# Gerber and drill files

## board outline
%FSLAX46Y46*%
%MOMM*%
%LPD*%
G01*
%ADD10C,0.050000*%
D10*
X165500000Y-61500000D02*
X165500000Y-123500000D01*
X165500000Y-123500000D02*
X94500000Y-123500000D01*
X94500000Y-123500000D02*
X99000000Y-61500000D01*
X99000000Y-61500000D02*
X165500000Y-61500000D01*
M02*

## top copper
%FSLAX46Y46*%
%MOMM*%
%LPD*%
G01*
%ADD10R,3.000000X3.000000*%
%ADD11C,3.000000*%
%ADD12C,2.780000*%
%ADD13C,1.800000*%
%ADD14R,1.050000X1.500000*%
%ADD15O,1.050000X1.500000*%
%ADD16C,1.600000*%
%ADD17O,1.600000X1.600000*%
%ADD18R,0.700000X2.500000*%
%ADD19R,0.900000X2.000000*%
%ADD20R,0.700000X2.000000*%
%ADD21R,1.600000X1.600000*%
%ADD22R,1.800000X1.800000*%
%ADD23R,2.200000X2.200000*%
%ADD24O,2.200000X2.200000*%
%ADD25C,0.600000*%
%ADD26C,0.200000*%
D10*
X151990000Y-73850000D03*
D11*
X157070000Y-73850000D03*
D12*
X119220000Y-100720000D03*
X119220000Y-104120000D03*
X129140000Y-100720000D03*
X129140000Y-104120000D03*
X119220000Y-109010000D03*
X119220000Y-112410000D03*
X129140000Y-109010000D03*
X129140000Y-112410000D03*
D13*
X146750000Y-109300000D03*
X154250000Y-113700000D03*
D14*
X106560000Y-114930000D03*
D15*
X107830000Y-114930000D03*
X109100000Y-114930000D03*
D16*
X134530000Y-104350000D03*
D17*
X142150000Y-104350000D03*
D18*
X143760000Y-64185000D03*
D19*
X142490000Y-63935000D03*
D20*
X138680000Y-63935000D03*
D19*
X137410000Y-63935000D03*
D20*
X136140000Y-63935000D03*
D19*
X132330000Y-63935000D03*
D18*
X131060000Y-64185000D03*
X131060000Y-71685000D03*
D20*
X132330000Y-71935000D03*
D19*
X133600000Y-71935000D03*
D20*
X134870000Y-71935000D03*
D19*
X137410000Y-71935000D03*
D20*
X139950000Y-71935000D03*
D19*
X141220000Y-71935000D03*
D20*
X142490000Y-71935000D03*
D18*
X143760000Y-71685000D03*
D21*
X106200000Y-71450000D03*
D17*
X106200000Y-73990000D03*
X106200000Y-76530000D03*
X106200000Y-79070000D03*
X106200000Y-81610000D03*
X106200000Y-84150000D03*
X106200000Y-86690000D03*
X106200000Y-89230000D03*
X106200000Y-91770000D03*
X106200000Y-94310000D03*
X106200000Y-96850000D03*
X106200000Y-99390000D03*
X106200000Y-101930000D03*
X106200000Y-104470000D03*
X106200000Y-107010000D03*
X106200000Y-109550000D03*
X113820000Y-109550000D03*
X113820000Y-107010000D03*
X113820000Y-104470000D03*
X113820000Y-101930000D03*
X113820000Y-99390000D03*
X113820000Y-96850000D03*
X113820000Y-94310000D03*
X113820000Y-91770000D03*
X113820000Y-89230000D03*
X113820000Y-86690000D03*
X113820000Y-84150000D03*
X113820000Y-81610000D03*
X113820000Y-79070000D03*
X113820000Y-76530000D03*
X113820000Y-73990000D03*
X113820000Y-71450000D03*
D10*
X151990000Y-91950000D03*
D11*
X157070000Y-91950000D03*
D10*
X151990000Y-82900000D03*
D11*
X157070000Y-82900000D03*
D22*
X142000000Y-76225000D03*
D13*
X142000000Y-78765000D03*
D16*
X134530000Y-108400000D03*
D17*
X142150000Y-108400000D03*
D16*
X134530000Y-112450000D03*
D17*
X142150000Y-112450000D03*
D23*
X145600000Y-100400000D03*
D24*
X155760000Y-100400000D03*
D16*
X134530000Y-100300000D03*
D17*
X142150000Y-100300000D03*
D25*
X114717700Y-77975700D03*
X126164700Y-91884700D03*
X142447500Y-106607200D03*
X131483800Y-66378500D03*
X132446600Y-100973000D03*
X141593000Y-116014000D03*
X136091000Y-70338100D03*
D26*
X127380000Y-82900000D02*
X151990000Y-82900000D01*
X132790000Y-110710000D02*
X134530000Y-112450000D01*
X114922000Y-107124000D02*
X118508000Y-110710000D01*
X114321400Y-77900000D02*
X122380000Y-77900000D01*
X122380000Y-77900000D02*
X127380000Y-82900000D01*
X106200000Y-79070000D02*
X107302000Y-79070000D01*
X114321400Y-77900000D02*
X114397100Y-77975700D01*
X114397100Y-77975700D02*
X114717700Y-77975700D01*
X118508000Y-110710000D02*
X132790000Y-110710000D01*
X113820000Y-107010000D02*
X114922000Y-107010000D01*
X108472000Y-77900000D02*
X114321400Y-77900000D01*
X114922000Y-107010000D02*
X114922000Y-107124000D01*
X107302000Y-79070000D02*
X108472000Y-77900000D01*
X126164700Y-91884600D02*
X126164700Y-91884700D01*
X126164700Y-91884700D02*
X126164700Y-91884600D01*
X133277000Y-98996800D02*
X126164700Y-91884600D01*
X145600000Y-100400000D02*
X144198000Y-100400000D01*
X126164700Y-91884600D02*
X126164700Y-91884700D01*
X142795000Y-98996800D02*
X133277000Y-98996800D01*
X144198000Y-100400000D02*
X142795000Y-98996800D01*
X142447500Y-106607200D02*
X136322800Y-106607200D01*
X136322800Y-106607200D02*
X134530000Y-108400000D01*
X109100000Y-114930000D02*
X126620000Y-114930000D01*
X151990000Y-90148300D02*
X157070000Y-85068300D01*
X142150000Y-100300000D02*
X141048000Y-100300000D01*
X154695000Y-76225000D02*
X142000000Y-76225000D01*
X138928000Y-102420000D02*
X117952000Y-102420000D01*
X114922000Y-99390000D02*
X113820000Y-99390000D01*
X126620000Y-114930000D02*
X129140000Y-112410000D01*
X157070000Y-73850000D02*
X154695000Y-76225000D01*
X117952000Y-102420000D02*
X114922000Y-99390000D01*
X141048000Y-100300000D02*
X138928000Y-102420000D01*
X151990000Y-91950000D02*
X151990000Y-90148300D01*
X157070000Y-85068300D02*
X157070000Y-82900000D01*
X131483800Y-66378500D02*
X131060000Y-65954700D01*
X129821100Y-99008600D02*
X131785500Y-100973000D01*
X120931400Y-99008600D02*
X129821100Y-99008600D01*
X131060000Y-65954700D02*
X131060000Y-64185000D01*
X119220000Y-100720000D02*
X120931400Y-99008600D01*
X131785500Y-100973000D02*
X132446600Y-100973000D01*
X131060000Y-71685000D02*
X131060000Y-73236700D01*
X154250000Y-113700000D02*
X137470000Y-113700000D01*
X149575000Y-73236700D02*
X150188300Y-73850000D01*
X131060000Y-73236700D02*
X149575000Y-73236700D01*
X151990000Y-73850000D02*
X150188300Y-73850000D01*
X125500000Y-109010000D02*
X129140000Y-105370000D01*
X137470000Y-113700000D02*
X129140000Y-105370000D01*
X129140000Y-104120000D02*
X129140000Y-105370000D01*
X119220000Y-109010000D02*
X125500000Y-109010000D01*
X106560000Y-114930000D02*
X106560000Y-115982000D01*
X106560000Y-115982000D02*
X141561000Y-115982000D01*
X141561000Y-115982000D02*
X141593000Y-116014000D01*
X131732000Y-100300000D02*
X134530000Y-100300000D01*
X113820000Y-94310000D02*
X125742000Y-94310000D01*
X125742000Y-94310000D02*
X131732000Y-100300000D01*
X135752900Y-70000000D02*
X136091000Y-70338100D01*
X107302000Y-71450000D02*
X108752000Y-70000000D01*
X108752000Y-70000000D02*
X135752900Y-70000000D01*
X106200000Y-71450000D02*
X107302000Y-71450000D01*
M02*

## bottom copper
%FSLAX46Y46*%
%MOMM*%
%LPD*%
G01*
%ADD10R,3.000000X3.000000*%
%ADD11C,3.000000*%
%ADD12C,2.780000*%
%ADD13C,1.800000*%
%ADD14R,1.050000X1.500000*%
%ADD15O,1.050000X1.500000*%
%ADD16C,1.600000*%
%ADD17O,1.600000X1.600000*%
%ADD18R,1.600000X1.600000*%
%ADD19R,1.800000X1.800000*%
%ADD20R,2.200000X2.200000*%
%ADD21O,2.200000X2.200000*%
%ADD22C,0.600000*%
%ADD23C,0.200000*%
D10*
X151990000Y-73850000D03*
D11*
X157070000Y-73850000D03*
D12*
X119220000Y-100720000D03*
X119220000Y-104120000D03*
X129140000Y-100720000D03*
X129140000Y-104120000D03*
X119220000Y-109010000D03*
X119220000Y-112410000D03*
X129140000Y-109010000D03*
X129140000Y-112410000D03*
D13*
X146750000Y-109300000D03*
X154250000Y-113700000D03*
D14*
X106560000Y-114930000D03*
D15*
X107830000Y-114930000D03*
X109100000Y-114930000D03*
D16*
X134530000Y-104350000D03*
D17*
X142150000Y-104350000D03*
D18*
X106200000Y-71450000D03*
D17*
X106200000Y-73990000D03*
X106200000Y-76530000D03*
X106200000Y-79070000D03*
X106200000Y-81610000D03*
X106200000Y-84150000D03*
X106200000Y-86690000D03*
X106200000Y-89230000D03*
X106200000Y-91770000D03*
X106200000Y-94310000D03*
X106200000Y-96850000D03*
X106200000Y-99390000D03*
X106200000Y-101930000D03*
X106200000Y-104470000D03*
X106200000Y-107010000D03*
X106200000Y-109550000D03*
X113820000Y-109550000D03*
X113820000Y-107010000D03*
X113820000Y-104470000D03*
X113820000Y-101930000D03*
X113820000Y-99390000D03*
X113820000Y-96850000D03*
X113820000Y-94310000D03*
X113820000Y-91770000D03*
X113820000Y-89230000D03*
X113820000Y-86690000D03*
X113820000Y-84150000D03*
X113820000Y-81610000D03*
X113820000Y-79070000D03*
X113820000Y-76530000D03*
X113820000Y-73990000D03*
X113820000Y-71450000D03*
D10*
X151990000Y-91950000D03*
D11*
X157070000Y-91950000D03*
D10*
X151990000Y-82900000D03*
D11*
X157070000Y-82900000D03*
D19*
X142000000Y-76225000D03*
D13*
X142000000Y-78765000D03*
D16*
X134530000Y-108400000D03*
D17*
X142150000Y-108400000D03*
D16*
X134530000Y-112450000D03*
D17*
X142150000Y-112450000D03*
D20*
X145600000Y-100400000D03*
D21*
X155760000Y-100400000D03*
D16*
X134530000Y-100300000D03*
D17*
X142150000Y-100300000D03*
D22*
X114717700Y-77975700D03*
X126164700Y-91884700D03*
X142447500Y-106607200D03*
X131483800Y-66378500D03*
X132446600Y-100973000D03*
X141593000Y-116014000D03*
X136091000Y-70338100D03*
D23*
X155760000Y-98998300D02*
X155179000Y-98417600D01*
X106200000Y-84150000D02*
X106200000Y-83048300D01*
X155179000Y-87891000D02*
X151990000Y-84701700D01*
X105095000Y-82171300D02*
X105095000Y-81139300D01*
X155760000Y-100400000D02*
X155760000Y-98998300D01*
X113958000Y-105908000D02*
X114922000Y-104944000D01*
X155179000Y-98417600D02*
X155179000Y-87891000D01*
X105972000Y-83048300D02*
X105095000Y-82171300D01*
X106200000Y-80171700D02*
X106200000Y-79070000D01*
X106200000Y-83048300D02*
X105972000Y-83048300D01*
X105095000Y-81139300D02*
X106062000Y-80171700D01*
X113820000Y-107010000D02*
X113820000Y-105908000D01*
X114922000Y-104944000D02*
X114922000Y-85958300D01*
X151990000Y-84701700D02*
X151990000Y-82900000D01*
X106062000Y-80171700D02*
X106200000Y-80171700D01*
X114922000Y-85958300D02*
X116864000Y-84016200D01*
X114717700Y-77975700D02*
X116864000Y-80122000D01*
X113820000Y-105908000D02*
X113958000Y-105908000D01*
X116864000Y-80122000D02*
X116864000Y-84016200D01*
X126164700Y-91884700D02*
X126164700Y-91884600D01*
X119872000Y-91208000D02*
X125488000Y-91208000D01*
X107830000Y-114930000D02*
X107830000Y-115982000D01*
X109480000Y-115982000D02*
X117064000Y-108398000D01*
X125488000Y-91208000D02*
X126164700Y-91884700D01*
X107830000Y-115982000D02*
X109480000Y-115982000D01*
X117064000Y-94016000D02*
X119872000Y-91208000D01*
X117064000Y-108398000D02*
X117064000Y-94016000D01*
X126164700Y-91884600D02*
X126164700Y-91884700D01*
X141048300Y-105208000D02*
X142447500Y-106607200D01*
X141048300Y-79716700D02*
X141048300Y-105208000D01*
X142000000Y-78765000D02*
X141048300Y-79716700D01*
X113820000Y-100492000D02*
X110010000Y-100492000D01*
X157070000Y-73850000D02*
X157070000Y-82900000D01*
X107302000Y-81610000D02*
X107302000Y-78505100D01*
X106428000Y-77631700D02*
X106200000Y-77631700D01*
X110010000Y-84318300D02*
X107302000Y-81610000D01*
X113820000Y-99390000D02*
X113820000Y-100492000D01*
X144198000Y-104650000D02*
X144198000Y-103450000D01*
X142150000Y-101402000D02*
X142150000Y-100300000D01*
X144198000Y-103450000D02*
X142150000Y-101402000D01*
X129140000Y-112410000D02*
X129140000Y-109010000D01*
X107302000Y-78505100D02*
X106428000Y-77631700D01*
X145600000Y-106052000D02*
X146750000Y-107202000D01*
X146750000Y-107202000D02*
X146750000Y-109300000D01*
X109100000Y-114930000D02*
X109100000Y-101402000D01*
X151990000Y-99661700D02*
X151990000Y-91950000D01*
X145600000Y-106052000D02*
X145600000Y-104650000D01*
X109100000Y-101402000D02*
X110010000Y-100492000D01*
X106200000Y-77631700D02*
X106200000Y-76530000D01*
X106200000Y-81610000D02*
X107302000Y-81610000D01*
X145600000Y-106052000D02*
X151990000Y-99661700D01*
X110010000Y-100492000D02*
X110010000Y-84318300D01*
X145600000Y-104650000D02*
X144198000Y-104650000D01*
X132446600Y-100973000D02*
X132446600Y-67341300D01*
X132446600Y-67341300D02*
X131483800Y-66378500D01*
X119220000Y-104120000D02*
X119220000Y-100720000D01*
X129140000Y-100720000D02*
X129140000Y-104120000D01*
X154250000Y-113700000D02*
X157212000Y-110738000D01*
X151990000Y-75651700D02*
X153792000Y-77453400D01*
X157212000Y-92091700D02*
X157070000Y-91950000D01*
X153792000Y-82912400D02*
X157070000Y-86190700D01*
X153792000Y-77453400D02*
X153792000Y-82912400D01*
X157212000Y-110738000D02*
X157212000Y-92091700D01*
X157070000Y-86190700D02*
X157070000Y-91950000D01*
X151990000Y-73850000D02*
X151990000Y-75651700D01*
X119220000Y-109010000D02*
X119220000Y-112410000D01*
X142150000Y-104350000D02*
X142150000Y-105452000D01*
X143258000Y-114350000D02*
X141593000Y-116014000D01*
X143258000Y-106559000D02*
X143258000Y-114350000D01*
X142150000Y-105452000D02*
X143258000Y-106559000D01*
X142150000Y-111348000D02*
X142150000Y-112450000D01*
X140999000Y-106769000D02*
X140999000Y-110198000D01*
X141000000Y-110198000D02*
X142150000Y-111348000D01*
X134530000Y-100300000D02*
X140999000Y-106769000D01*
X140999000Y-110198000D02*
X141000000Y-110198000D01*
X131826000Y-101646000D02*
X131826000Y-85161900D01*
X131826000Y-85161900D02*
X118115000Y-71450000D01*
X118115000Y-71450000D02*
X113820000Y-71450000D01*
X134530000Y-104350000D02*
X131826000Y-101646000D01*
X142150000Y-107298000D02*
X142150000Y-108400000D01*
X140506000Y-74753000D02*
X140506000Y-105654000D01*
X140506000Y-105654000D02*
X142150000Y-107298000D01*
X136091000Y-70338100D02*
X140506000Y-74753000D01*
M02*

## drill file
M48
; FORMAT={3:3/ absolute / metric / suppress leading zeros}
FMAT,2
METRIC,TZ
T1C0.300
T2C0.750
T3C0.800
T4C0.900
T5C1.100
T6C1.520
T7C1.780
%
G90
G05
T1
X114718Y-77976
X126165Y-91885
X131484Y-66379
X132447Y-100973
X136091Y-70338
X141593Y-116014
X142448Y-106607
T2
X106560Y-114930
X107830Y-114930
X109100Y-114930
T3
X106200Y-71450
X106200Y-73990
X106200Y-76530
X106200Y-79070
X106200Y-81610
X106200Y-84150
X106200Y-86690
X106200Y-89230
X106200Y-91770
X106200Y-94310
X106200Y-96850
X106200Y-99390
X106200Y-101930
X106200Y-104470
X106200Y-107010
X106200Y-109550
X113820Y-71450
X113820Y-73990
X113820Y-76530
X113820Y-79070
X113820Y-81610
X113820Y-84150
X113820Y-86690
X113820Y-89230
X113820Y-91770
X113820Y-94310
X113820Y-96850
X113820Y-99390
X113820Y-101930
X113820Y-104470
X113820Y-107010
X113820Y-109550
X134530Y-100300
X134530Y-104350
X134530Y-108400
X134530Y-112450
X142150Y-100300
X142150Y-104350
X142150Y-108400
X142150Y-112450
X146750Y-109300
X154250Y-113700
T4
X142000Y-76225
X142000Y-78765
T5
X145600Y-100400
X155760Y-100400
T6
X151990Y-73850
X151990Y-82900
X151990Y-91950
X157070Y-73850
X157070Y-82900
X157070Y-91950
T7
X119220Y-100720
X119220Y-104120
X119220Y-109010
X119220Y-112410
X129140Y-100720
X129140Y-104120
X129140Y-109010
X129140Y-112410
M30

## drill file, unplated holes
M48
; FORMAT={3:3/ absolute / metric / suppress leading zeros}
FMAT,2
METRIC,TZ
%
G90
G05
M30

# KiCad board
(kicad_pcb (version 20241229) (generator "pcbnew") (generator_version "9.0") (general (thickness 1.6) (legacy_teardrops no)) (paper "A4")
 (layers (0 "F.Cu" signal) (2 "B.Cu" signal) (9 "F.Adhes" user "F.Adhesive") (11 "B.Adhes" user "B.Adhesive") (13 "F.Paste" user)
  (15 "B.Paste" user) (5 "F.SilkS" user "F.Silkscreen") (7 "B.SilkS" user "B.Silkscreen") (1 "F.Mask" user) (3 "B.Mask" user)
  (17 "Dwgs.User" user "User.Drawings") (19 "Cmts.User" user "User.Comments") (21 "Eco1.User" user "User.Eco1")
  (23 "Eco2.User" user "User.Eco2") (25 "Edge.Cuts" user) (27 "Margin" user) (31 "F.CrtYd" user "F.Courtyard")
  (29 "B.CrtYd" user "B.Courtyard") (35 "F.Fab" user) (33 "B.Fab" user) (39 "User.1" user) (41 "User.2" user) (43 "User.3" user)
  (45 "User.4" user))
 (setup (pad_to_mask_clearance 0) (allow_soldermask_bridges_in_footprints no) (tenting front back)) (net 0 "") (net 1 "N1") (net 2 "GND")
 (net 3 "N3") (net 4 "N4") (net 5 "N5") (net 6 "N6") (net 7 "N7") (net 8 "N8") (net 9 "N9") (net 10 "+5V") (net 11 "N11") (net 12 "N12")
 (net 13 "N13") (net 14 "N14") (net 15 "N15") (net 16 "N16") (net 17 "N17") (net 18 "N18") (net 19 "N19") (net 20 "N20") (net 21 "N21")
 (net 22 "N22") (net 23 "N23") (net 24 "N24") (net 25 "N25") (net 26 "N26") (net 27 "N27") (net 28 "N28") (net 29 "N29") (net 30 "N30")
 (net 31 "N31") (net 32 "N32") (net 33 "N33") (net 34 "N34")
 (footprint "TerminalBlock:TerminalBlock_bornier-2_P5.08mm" (layer "F.Cu") (at 151.99 73.85)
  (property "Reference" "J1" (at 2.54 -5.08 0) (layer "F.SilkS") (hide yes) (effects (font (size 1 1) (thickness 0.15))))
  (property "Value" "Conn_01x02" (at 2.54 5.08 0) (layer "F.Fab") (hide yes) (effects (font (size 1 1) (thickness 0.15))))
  (pad "1" thru_hole rect (at 0 0) (size 3 3) (drill 1.52) (layers "*.Cu" "*.Mask") (remove_unused_layers no) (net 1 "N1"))
  (pad "2" thru_hole circle (at 5.08 0) (size 3 3) (drill 1.52) (layers "*.Cu" "*.Mask") (remove_unused_layers no) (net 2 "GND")))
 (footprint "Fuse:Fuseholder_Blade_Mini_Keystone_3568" (layer "F.Cu") (at 119.22 100.72)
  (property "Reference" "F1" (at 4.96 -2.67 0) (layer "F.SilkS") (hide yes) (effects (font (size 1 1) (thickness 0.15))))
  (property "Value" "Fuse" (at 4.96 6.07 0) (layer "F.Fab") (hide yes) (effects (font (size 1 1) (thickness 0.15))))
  (pad "1" thru_hole circle (at 0 0) (size 2.78 2.78) (drill 1.78) (layers "*.Cu" "*.Mask") (remove_unused_layers no) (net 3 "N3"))
  (pad "1" thru_hole circle (at 0 3.4) (size 2.78 2.78) (drill 1.78) (layers "*.Cu" "*.Mask") (remove_unused_layers no) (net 3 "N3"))
  (pad "2" thru_hole circle (at 9.92 0) (size 2.78 2.78) (drill 1.78) (layers "*.Cu" "*.Mask") (remove_unused_layers no) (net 1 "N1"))
  (pad "2" thru_hole circle (at 9.92 3.4) (size 2.78 2.78) (drill 1.78) (layers "*.Cu" "*.Mask") (remove_unused_layers no) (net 1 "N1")))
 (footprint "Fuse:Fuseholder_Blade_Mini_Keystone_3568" (layer "F.Cu") (at 119.22 109.01)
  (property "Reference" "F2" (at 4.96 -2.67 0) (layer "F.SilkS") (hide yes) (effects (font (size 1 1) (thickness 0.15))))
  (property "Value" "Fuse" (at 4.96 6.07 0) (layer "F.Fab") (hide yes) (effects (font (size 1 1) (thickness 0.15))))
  (pad "1" thru_hole circle (at 0 0) (size 2.78 2.78) (drill 1.78) (layers "*.Cu" "*.Mask") (remove_unused_layers no) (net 1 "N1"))
  (pad "1" thru_hole circle (at 0 3.4) (size 2.78 2.78) (drill 1.78) (layers "*.Cu" "*.Mask") (remove_unused_layers no) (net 1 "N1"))
  (pad "2" thru_hole circle (at 9.92 0) (size 2.78 2.78) (drill 1.78) (layers "*.Cu" "*.Mask") (remove_unused_layers no) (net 2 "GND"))
  (pad "2" thru_hole circle (at 9.92 3.4) (size 2.78 2.78) (drill 1.78) (layers "*.Cu" "*.Mask") (remove_unused_layers no) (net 2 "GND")))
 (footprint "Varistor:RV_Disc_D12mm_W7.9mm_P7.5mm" (layer "F.Cu") (at 146.75 109.3)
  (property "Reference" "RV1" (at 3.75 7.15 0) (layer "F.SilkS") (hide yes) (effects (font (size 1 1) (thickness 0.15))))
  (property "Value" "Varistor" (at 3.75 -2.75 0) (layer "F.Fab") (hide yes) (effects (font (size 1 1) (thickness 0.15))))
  (pad "1" thru_hole circle (at 0 0) (size 1.8 1.8) (drill 0.8) (layers "*.Cu" "*.Mask") (remove_unused_layers no) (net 2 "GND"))
  (pad "2" thru_hole circle (at 7.5 4.4) (size 1.8 1.8) (drill 0.8) (layers "*.Cu" "*.Mask") (remove_unused_layers no) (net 1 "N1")))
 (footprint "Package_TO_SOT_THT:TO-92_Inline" (layer "F.Cu") (at 106.56 114.93)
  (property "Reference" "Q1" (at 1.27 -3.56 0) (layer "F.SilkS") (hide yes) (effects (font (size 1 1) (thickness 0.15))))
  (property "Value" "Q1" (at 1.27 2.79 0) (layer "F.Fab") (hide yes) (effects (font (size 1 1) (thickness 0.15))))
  (pad "1" thru_hole rect (at 0 0) (size 1.05 1.5) (drill 0.75) (layers "*.Cu" "*.Mask") (remove_unused_layers no) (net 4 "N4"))
  (pad "2" thru_hole oval (at 1.27 0) (size 1.05 1.5) (drill 0.75) (layers "*.Cu" "*.Mask") (remove_unused_layers no) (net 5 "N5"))
  (pad "3" thru_hole oval (at 2.54 0) (size 1.05 1.5) (drill 0.75) (layers "*.Cu" "*.Mask") (remove_unused_layers no) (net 2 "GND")))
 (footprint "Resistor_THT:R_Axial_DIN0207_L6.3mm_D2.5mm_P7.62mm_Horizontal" (layer "F.Cu") (at 134.53 104.35)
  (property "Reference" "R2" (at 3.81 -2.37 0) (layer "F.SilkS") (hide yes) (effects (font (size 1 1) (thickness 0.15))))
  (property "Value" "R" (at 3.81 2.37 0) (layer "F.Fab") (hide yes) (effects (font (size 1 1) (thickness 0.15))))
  (pad "1" thru_hole circle (at 0 0) (size 1.6 1.6) (drill 0.8) (layers "*.Cu" "*.Mask") (remove_unused_layers no) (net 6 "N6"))
  (pad "2" thru_hole oval (at 7.62 0) (size 1.6 1.6) (drill 0.8) (layers "*.Cu" "*.Mask") (remove_unused_layers no) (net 4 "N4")))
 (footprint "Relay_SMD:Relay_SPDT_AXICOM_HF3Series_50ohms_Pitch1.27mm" (layer "F.Cu") (at 137.41 67.935 -90)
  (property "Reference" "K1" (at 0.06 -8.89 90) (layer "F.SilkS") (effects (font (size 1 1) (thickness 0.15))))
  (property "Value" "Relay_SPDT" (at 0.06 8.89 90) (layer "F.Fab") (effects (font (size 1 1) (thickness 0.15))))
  (pad "1" smd rect (at -3.75 -6.35 270) (size 2.5 0.7) (layers "F.Cu" "F.Mask" "F.Paste"))
  (pad "2" smd rect (at -4 -5.08 270) (size 2 0.9) (layers "F.Cu" "F.Mask" "F.Paste"))
  (pad "5" smd rect (at -4 -1.27 270) (size 2 0.7) (layers "F.Cu" "F.Mask" "F.Paste"))
  (pad "6" smd rect (at -4 0 270) (size 2 0.9) (layers "F.Cu" "F.Mask" "F.Paste"))
  (pad "7" smd rect (at -4 1.27 270) (size 2 0.7) (layers "F.Cu" "F.Mask" "F.Paste"))
  (pad "10" smd rect (at -4 5.08 270) (size 2 0.9) (layers "F.Cu" "F.Mask" "F.Paste"))
  (pad "11" smd rect (at -3.75 6.35 270) (size 2.5 0.7) (layers "F.Cu" "F.Mask" "F.Paste") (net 3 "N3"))
  (pad "12" smd rect (at 3.75 6.35 270) (size 2.5 0.7) (layers "F.Cu" "F.Mask" "F.Paste") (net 1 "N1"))
  (pad "13" smd rect (at 4 5.08 270) (size 2 0.7) (layers "F.Cu" "F.Mask" "F.Paste"))
  (pad "14" smd rect (at 4 3.81 270) (size 2 0.9) (layers "F.Cu" "F.Mask" "F.Paste") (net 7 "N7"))
  (pad "15" smd rect (at 4 2.54 270) (size 2 0.7) (layers "F.Cu" "F.Mask" "F.Paste"))
  (pad "17" smd rect (at 4 0 270) (size 2 0.9) (layers "F.Cu" "F.Mask" "F.Paste"))
  (pad "19" smd rect (at 4 -2.54 270) (size 2 0.7) (layers "F.Cu" "F.Mask" "F.Paste"))
  (pad "20" smd rect (at 4 -3.81 270) (size 2 0.9) (layers "F.Cu" "F.Mask" "F.Paste"))
  (pad "21" smd rect (at 4 -5.08 270) (size 2 0.7) (layers "F.Cu" "F.Mask" "F.Paste"))
  (pad "22" smd rect (at 3.75 -6.35 270) (size 2.5 0.7) (layers "F.Cu" "F.Mask" "F.Paste")))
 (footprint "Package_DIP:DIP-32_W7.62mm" (layer "F.Cu") (at 106.2 71.45)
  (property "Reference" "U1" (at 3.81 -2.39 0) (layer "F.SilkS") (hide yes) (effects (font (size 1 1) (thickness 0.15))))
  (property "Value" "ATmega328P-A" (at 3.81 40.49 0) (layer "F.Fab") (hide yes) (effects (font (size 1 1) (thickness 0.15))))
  (pad "1" thru_hole rect (at 0 0) (size 1.6 1.6) (drill 0.8) (layers "*.Cu" "*.Mask") (remove_unused_layers no) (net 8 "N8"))
  (pad "2" thru_hole oval (at 0 2.54) (size 1.6 1.6) (drill 0.8) (layers "*.Cu" "*.Mask") (remove_unused_layers no) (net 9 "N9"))
  (pad "3" thru_hole oval (at 0 5.08) (size 1.6 1.6) (drill 0.8) (layers "*.Cu" "*.Mask") (remove_unused_layers no) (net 2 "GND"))
  (pad "4" thru_hole oval (at 0 7.62) (size 1.6 1.6) (drill 0.8) (layers "*.Cu" "*.Mask") (remove_unused_layers no) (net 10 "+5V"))
  (pad "5" thru_hole oval (at 0 10.16) (size 1.6 1.6) (drill 0.8) (layers "*.Cu" "*.Mask") (remove_unused_layers no) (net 2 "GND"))
  (pad "6" thru_hole oval (at 0 12.7) (size 1.6 1.6) (drill 0.8) (layers "*.Cu" "*.Mask") (remove_unused_layers no) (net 10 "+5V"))
  (pad "7" thru_hole oval (at 0 15.24) (size 1.6 1.6) (drill 0.8) (layers "*.Cu" "*.Mask") (remove_unused_layers no) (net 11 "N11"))
  (pad "8" thru_hole oval (at 0 17.78) (size 1.6 1.6) (drill 0.8) (layers "*.Cu" "*.Mask") (remove_unused_layers no) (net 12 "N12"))
  (pad "9" thru_hole oval (at 0 20.32) (size 1.6 1.6) (drill 0.8) (layers "*.Cu" "*.Mask") (remove_unused_layers no) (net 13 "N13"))
  (pad "10" thru_hole oval (at 0 22.86) (size 1.6 1.6) (drill 0.8) (layers "*.Cu" "*.Mask") (remove_unused_layers no) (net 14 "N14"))
  (pad "11" thru_hole oval (at 0 25.4) (size 1.6 1.6) (drill 0.8) (layers "*.Cu" "*.Mask") (remove_unused_layers no) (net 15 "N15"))
  (pad "12" thru_hole oval (at 0 27.94) (size 1.6 1.6) (drill 0.8) (layers "*.Cu" "*.Mask") (remove_unused_layers no) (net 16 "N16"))
  (pad "13" thru_hole oval (at 0 30.48) (size 1.6 1.6) (drill 0.8) (layers "*.Cu" "*.Mask") (remove_unused_layers no) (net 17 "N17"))
  (pad "14" thru_hole oval (at 0 33.02) (size 1.6 1.6) (drill 0.8) (layers "*.Cu" "*.Mask") (remove_unused_layers no) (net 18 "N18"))
  (pad "15" thru_hole oval (at 0 35.56) (size 1.6 1.6) (drill 0.8) (layers "*.Cu" "*.Mask") (remove_unused_layers no) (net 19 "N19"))
  (pad "16" thru_hole oval (at 0 38.1) (size 1.6 1.6) (drill 0.8) (layers "*.Cu" "*.Mask") (remove_unused_layers no) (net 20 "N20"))
  (pad "17" thru_hole oval (at 7.62 38.1) (size 1.6 1.6) (drill 0.8) (layers "*.Cu" "*.Mask") (remove_unused_layers no) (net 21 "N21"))
  (pad "18" thru_hole oval (at 7.62 35.56) (size 1.6 1.6) (drill 0.8) (layers "*.Cu" "*.Mask") (remove_unused_layers no) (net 10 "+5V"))
  (pad "19" thru_hole oval (at 7.62 33.02) (size 1.6 1.6) (drill 0.8) (layers "*.Cu" "*.Mask") (remove_unused_layers no) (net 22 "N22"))
  (pad "20" thru_hole oval (at 7.62 30.48) (size 1.6 1.6) (drill 0.8) (layers "*.Cu" "*.Mask") (remove_unused_layers no) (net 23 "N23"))
  (pad "21" thru_hole oval (at 7.62 27.94) (size 1.6 1.6) (drill 0.8) (layers "*.Cu" "*.Mask") (remove_unused_layers no) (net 2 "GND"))
  (pad "22" thru_hole oval (at 7.62 25.4) (size 1.6 1.6) (drill 0.8) (layers "*.Cu" "*.Mask") (remove_unused_layers no) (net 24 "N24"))
  (pad "23" thru_hole oval (at 7.62 22.86) (size 1.6 1.6) (drill 0.8) (layers "*.Cu" "*.Mask") (remove_unused_layers no) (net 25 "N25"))
  (pad "24" thru_hole oval (at 7.62 20.32) (size 1.6 1.6) (drill 0.8) (layers "*.Cu" "*.Mask") (remove_unused_layers no) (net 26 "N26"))
  (pad "25" thru_hole oval (at 7.62 17.78) (size 1.6 1.6) (drill 0.8) (layers "*.Cu" "*.Mask") (remove_unused_layers no) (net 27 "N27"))
  (pad "26" thru_hole oval (at 7.62 15.24) (size 1.6 1.6) (drill 0.8) (layers "*.Cu" "*.Mask") (remove_unused_layers no) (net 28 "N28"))
  (pad "27" thru_hole oval (at 7.62 12.7) (size 1.6 1.6) (drill 0.8) (layers "*.Cu" "*.Mask") (remove_unused_layers no) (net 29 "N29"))
  (pad "28" thru_hole oval (at 7.62 10.16) (size 1.6 1.6) (drill 0.8) (layers "*.Cu" "*.Mask") (remove_unused_layers no) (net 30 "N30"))
  (pad "29" thru_hole oval (at 7.62 7.62) (size 1.6 1.6) (drill 0.8) (layers "*.Cu" "*.Mask") (remove_unused_layers no) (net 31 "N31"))
  (pad "30" thru_hole oval (at 7.62 5.08) (size 1.6 1.6) (drill 0.8) (layers "*.Cu" "*.Mask") (remove_unused_layers no) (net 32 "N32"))
  (pad "31" thru_hole oval (at 7.62 2.54) (size 1.6 1.6) (drill 0.8) (layers "*.Cu" "*.Mask") (remove_unused_layers no) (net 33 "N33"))
  (pad "32" thru_hole oval (at 7.62 0) (size 1.6 1.6) (drill 0.8) (layers "*.Cu" "*.Mask") (remove_unused_layers no) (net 6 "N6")))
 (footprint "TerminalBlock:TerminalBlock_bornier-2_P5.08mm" (layer "F.Cu") (at 151.99 91.95)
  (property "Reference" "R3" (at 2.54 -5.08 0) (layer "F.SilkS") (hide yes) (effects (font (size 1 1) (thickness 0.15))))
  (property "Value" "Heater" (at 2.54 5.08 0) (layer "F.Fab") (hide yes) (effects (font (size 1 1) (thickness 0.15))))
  (pad "1" thru_hole rect (at 0 0) (size 3 3) (drill 1.52) (layers "*.Cu" "*.Mask") (remove_unused_layers no) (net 2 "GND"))
  (pad "2" thru_hole circle (at 5.08 0) (size 3 3) (drill 1.52) (layers "*.Cu" "*.Mask") (remove_unused_layers no) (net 1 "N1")))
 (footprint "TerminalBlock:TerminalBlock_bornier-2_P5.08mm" (layer "F.Cu") (at 151.99 82.9)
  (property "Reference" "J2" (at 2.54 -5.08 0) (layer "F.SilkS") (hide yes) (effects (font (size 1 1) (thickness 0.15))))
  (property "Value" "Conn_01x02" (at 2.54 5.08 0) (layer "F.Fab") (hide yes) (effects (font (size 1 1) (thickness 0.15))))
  (pad "1" thru_hole rect (at 0 0) (size 3 3) (drill 1.52) (layers "*.Cu" "*.Mask") (remove_unused_layers no) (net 10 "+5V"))
  (pad "2" thru_hole circle (at 5.08 0) (size 3 3) (drill 1.52) (layers "*.Cu" "*.Mask") (remove_unused_layers no) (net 2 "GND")))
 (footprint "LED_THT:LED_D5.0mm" (layer "F.Cu") (at 142 76.225 -90)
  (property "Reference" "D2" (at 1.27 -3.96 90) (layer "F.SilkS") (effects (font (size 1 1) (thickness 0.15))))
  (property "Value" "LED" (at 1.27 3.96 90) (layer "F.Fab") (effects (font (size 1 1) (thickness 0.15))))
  (pad "1" thru_hole rect (at 0 0 270) (size 1.8 1.8) (drill 0.9) (layers "*.Cu" "*.Mask") (remove_unused_layers no) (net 2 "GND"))
  (pad "2" thru_hole circle (at 2.54 0 270) (size 1.8 1.8) (drill 0.9) (layers "*.Cu" "*.Mask") (remove_unused_layers no) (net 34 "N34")))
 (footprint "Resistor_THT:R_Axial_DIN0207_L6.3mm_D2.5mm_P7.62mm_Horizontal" (layer "F.Cu") (at 134.53 108.4)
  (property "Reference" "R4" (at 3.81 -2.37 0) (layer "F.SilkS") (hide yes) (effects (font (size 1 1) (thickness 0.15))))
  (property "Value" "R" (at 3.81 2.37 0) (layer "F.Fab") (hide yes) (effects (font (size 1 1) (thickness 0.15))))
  (pad "1" thru_hole circle (at 0 0) (size 1.6 1.6) (drill 0.8) (layers "*.Cu" "*.Mask") (remove_unused_layers no) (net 34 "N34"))
  (pad "2" thru_hole oval (at 7.62 0) (size 1.6 1.6) (drill 0.8) (layers "*.Cu" "*.Mask") (remove_unused_layers no) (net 8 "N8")))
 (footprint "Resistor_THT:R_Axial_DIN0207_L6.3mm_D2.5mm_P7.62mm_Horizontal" (layer "F.Cu") (at 134.53 112.45)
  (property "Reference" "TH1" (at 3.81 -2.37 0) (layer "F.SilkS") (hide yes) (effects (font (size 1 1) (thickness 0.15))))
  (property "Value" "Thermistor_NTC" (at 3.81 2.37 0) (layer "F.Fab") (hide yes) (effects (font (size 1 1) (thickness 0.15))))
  (pad "1" thru_hole circle (at 0 0) (size 1.6 1.6) (drill 0.8) (layers "*.Cu" "*.Mask") (remove_unused_layers no) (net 10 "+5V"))
  (pad "2" thru_hole oval (at 7.62 0) (size 1.6 1.6) (drill 0.8) (layers "*.Cu" "*.Mask") (remove_unused_layers no) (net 25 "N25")))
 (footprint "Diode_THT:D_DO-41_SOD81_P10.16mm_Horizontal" (layer "F.Cu") (at 145.6 100.4)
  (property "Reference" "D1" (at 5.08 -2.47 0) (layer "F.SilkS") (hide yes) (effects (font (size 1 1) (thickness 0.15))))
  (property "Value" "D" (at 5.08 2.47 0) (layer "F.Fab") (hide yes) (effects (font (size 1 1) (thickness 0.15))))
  (pad "1" thru_hole rect (at 0 0) (size 2.2 2.2) (drill 1.1) (layers "*.Cu" "*.Mask") (remove_unused_layers no) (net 5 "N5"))
  (pad "2" thru_hole oval (at 10.16 0) (size 2.2 2.2) (drill 1.1) (layers "*.Cu" "*.Mask") (remove_unused_layers no) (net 10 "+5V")))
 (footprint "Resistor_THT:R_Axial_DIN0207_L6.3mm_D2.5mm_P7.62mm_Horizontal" (layer "F.Cu") (at 134.53 100.3)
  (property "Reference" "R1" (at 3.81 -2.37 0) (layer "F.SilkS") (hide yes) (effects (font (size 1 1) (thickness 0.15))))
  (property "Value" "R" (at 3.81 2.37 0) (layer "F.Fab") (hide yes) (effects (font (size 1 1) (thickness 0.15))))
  (pad "1" thru_hole circle (at 0 0) (size 1.6 1.6) (drill 0.8) (layers "*.Cu" "*.Mask") (remove_unused_layers no) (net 25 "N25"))
  (pad "2" thru_hole oval (at 7.62 0) (size 1.6 1.6) (drill 0.8) (layers "*.Cu" "*.Mask") (remove_unused_layers no) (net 2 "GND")))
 (gr_line (start 165.5 61.5) (end 165.5 123.5) (stroke (width 0.05) (type default)) (layer "Edge.Cuts"))
 (gr_line (start 165.5 123.5) (end 94.5 123.5) (stroke (width 0.05) (type default)) (layer "Edge.Cuts"))
 (gr_line (start 94.5 123.5) (end 99 61.5) (stroke (width 0.05) (type default)) (layer "Edge.Cuts"))
 (gr_line (start 99 61.5) (end 165.5 61.5) (stroke (width 0.05) (type default)) (layer "Edge.Cuts"))
 (segment (start 127.38 82.9) (end 151.99 82.9) (width 0.2) (layer "F.Cu") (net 10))
 (segment (start 132.79 110.71) (end 134.53 112.45) (width 0.2) (layer "F.Cu") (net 10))
 (segment (start 114.922 107.124) (end 118.508 110.71) (width 0.2) (layer "F.Cu") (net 10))
 (segment (start 114.3214 77.9) (end 122.38 77.9) (width 0.2) (layer "F.Cu") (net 10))
 (segment (start 122.38 77.9) (end 127.38 82.9) (width 0.2) (layer "F.Cu") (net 10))
 (segment (start 106.2 79.07) (end 107.302 79.07) (width 0.2) (layer "F.Cu") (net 10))
 (segment (start 114.3214 77.9) (end 114.3971 77.9757) (width 0.2) (layer "F.Cu") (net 10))
 (segment (start 114.3971 77.9757) (end 114.7177 77.9757) (width 0.2) (layer "F.Cu") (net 10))
 (segment (start 118.508 110.71) (end 132.79 110.71) (width 0.2) (layer "F.Cu") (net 10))
 (segment (start 113.82 107.01) (end 114.922 107.01) (width 0.2) (layer "F.Cu") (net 10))
 (segment (start 108.472 77.9) (end 114.3214 77.9) (width 0.2) (layer "F.Cu") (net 10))
 (segment (start 114.922 107.01) (end 114.922 107.124) (width 0.2) (layer "F.Cu") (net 10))
 (segment (start 107.302 79.07) (end 108.472 77.9) (width 0.2) (layer "F.Cu") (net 10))
 (via (at 114.7177 77.9757) (size 0.6) (drill 0.3) (layers "F.Cu" "B.Cu") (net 10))
 (segment (start 155.76 98.9983) (end 155.179 98.4176) (width 0.2) (layer "B.Cu") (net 10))
 (segment (start 106.2 84.15) (end 106.2 83.0483) (width 0.2) (layer "B.Cu") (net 10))
 (segment (start 155.179 87.891) (end 151.99 84.7017) (width 0.2) (layer "B.Cu") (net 10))
 (segment (start 105.095 82.1713) (end 105.095 81.1393) (width 0.2) (layer "B.Cu") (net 10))
 (segment (start 155.76 100.4) (end 155.76 98.9983) (width 0.2) (layer "B.Cu") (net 10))
 (segment (start 113.958 105.908) (end 114.922 104.944) (width 0.2) (layer "B.Cu") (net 10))
 (segment (start 155.179 98.4176) (end 155.179 87.891) (width 0.2) (layer "B.Cu") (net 10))
 (segment (start 105.972 83.0483) (end 105.095 82.1713) (width 0.2) (layer "B.Cu") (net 10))
 (segment (start 106.2 80.1717) (end 106.2 79.07) (width 0.2) (layer "B.Cu") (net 10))
 (segment (start 106.2 83.0483) (end 105.972 83.0483) (width 0.2) (layer "B.Cu") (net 10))
 (segment (start 105.095 81.1393) (end 106.062 80.1717) (width 0.2) (layer "B.Cu") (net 10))
 (segment (start 113.82 107.01) (end 113.82 105.908) (width 0.2) (layer "B.Cu") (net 10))
 (segment (start 114.922 104.944) (end 114.922 85.9583) (width 0.2) (layer "B.Cu") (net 10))
 (segment (start 151.99 84.7017) (end 151.99 82.9) (width 0.2) (layer "B.Cu") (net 10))
 (segment (start 106.062 80.1717) (end 106.2 80.1717) (width 0.2) (layer "B.Cu") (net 10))
 (segment (start 114.922 85.9583) (end 116.864 84.0162) (width 0.2) (layer "B.Cu") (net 10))
 (segment (start 114.7177 77.9757) (end 116.864 80.122) (width 0.2) (layer "B.Cu") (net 10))
 (segment (start 113.82 105.908) (end 113.958 105.908) (width 0.2) (layer "B.Cu") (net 10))
 (segment (start 116.864 80.122) (end 116.864 84.0162) (width 0.2) (layer "B.Cu") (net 10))
 (segment (start 126.1647 91.8846) (end 126.1647 91.8847) (width 0.2) (layer "F.Cu") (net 5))
 (segment (start 126.1647 91.8847) (end 126.1647 91.8846) (width 0.2) (layer "F.Cu") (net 5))
 (segment (start 133.277 98.9968) (end 126.1647 91.8846) (width 0.2) (layer "F.Cu") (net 5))
 (segment (start 145.6 100.4) (end 144.198 100.4) (width 0.2) (layer "F.Cu") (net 5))
 (segment (start 126.1647 91.8846) (end 126.1647 91.8847) (width 0.2) (layer "F.Cu") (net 5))
 (segment (start 142.795 98.9968) (end 133.277 98.9968) (width 0.2) (layer "F.Cu") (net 5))
 (segment (start 144.198 100.4) (end 142.795 98.9968) (width 0.2) (layer "F.Cu") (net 5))
 (via (at 126.1647 91.8847) (size 0.6) (drill 0.3) (layers "F.Cu" "B.Cu") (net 5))
 (segment (start 126.1647 91.8847) (end 126.1647 91.8846) (width 0.2) (layer "B.Cu") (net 5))
 (segment (start 119.872 91.208) (end 125.488 91.208) (width 0.2) (layer "B.Cu") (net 5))
 (segment (start 107.83 114.93) (end 107.83 115.982) (width 0.2) (layer "B.Cu") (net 5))
 (segment (start 109.48 115.982) (end 117.064 108.398) (width 0.2) (layer "B.Cu") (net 5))
 (segment (start 125.488 91.208) (end 126.1647 91.8847) (width 0.2) (layer "B.Cu") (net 5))
 (segment (start 107.83 115.982) (end 109.48 115.982) (width 0.2) (layer "B.Cu") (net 5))
 (segment (start 117.064 94.016) (end 119.872 91.208) (width 0.2) (layer "B.Cu") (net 5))
 (segment (start 117.064 108.398) (end 117.064 94.016) (width 0.2) (layer "B.Cu") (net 5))
 (segment (start 126.1647 91.8846) (end 126.1647 91.8847) (width 0.2) (layer "B.Cu") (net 5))
 (segment (start 142.4475 106.6072) (end 136.3228 106.6072) (width 0.2) (layer "F.Cu") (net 34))
 (segment (start 136.3228 106.6072) (end 134.53 108.4) (width 0.2) (layer "F.Cu") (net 34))
 (via (at 142.4475 106.6072) (size 0.6) (drill 0.3) (layers "F.Cu" "B.Cu") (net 34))
 (segment (start 141.0483 105.208) (end 142.4475 106.6072) (width 0.2) (layer "B.Cu") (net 34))
 (segment (start 141.0483 79.7167) (end 141.0483 105.208) (width 0.2) (layer "B.Cu") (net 34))
 (segment (start 142 78.765) (end 141.0483 79.7167) (width 0.2) (layer "B.Cu") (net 34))
 (segment (start 109.1 114.93) (end 126.62 114.93) (width 0.2) (layer "F.Cu") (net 2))
 (segment (start 151.99 90.1483) (end 157.07 85.0683) (width 0.2) (layer "F.Cu") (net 2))
 (segment (start 142.15 100.3) (end 141.048 100.3) (width 0.2) (layer "F.Cu") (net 2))
 (segment (start 154.695 76.225) (end 142 76.225) (width 0.2) (layer "F.Cu") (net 2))
 (segment (start 138.928 102.42) (end 117.952 102.42) (width 0.2) (layer "F.Cu") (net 2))
 (segment (start 114.922 99.39) (end 113.82 99.39) (width 0.2) (layer "F.Cu") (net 2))
 (segment (start 126.62 114.93) (end 129.14 112.41) (width 0.2) (layer "F.Cu") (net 2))
 (segment (start 157.07 73.85) (end 154.695 76.225) (width 0.2) (layer "F.Cu") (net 2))
 (segment (start 117.952 102.42) (end 114.922 99.39) (width 0.2) (layer "F.Cu") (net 2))
 (segment (start 141.048 100.3) (end 138.928 102.42) (width 0.2) (layer "F.Cu") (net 2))
 (segment (start 151.99 91.95) (end 151.99 90.1483) (width 0.2) (layer "F.Cu") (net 2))
 (segment (start 157.07 85.0683) (end 157.07 82.9) (width 0.2) (layer "F.Cu") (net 2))
 (segment (start 113.82 100.492) (end 110.01 100.492) (width 0.2) (layer "B.Cu") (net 2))
 (segment (start 157.07 73.85) (end 157.07 82.9) (width 0.2) (layer "B.Cu") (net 2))
 (segment (start 107.302 81.61) (end 107.302 78.5051) (width 0.2) (layer "B.Cu") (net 2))
 (segment (start 106.428 77.6317) (end 106.2 77.6317) (width 0.2) (layer "B.Cu") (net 2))
 (segment (start 110.01 84.3183) (end 107.302 81.61) (width 0.2) (layer "B.Cu") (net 2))
 (segment (start 113.82 99.39) (end 113.82 100.492) (width 0.2) (layer "B.Cu") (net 2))
 (segment (start 144.198 104.65) (end 144.198 103.45) (width 0.2) (layer "B.Cu") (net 2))
 (segment (start 142.15 101.402) (end 142.15 100.3) (width 0.2) (layer "B.Cu") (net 2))
 (segment (start 144.198 103.45) (end 142.15 101.402) (width 0.2) (layer "B.Cu") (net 2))
 (segment (start 129.14 112.41) (end 129.14 109.01) (width 0.2) (layer "B.Cu") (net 2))
 (segment (start 107.302 78.5051) (end 106.428 77.6317) (width 0.2) (layer "B.Cu") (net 2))
 (segment (start 145.6 106.052) (end 146.75 107.202) (width 0.2) (layer "B.Cu") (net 2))
 (segment (start 146.75 107.202) (end 146.75 109.3) (width 0.2) (layer "B.Cu") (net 2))
 (segment (start 109.1 114.93) (end 109.1 101.402) (width 0.2) (layer "B.Cu") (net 2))
 (segment (start 151.99 99.6617) (end 151.99 91.95) (width 0.2) (layer "B.Cu") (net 2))
 (segment (start 145.6 106.052) (end 145.6 104.65) (width 0.2) (layer "B.Cu") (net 2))
 (segment (start 109.1 101.402) (end 110.01 100.492) (width 0.2) (layer "B.Cu") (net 2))
 (segment (start 106.2 77.6317) (end 106.2 76.53) (width 0.2) (layer "B.Cu") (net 2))
 (segment (start 106.2 81.61) (end 107.302 81.61) (width 0.2) (layer "B.Cu") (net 2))
 (segment (start 145.6 106.052) (end 151.99 99.6617) (width 0.2) (layer "B.Cu") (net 2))
 (segment (start 110.01 100.492) (end 110.01 84.3183) (width 0.2) (layer "B.Cu") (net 2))
 (segment (start 145.6 104.65) (end 144.198 104.65) (width 0.2) (layer "B.Cu") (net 2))
 (segment (start 131.4838 66.3785) (end 131.06 65.9547) (width 0.2) (layer "F.Cu") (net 3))
 (segment (start 129.8211 99.0086) (end 131.7855 100.973) (width 0.2) (layer "F.Cu") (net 3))
 (segment (start 120.9314 99.0086) (end 129.8211 99.0086) (width 0.2) (layer "F.Cu") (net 3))
 (segment (start 131.06 65.9547) (end 131.06 64.185) (width 0.2) (layer "F.Cu") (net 3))
 (segment (start 119.22 100.72) (end 120.9314 99.0086) (width 0.2) (layer "F.Cu") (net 3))
 (segment (start 131.7855 100.973) (end 132.4466 100.973) (width 0.2) (layer "F.Cu") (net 3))
 (via (at 131.4838 66.3785) (size 0.6) (drill 0.3) (layers "F.Cu" "B.Cu") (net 3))
 (via (at 132.4466 100.973) (size 0.6) (drill 0.3) (layers "F.Cu" "B.Cu") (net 3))
 (segment (start 132.4466 100.973) (end 132.4466 67.3413) (width 0.2) (layer "B.Cu") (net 3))
 (segment (start 132.4466 67.3413) (end 131.4838 66.3785) (width 0.2) (layer "B.Cu") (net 3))
 (segment (start 119.22 104.12) (end 119.22 100.72) (width 0.2) (layer "B.Cu") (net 3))
 (segment (start 131.06 71.685) (end 131.06 73.2367) (width 0.2) (layer "F.Cu") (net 1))
 (segment (start 154.25 113.7) (end 137.47 113.7) (width 0.2) (layer "F.Cu") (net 1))
 (segment (start 149.575 73.2367) (end 150.1883 73.85) (width 0.2) (layer "F.Cu") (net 1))
 (segment (start 131.06 73.2367) (end 149.575 73.2367) (width 0.2) (layer "F.Cu") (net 1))
 (segment (start 151.99 73.85) (end 150.1883 73.85) (width 0.2) (layer "F.Cu") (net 1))
 (segment (start 125.5 109.01) (end 129.14 105.37) (width 0.2) (layer "F.Cu") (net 1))
 (segment (start 137.47 113.7) (end 129.14 105.37) (width 0.2) (layer "F.Cu") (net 1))
 (segment (start 129.14 104.12) (end 129.14 105.37) (width 0.2) (layer "F.Cu") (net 1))
 (segment (start 119.22 109.01) (end 125.5 109.01) (width 0.2) (layer "F.Cu") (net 1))
 (segment (start 129.14 100.72) (end 129.14 104.12) (width 0.2) (layer "B.Cu") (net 1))
 (segment (start 154.25 113.7) (end 157.212 110.738) (width 0.2) (layer "B.Cu") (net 1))
 (segment (start 151.99 75.6517) (end 153.792 77.4534) (width 0.2) (layer "B.Cu") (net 1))
 (segment (start 157.212 92.0917) (end 157.07 91.95) (width 0.2) (layer "B.Cu") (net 1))
 (segment (start 153.792 82.9124) (end 157.07 86.1907) (width 0.2) (layer "B.Cu") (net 1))
 (segment (start 153.792 77.4534) (end 153.792 82.9124) (width 0.2) (layer "B.Cu") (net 1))
 (segment (start 157.212 110.738) (end 157.212 92.0917) (width 0.2) (layer "B.Cu") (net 1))
 (segment (start 157.07 86.1907) (end 157.07 91.95) (width 0.2) (layer "B.Cu") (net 1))
 (segment (start 151.99 73.85) (end 151.99 75.6517) (width 0.2) (layer "B.Cu") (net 1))
 (segment (start 119.22 109.01) (end 119.22 112.41) (width 0.2) (layer "B.Cu") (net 1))
 (segment (start 106.56 114.93) (end 106.56 115.982) (width 0.2) (layer "F.Cu") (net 4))
 (segment (start 106.56 115.982) (end 141.561 115.982) (width 0.2) (layer "F.Cu") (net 4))
 (segment (start 141.561 115.982) (end 141.593 116.014) (width 0.2) (layer "F.Cu") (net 4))
 (via (at 141.593 116.014) (size 0.6) (drill 0.3) (layers "F.Cu" "B.Cu") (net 4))
 (segment (start 142.15 104.35) (end 142.15 105.452) (width 0.2) (layer "B.Cu") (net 4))
 (segment (start 143.258 114.35) (end 141.593 116.014) (width 0.2) (layer "B.Cu") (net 4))
 (segment (start 143.258 106.559) (end 143.258 114.35) (width 0.2) (layer "B.Cu") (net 4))
 (segment (start 142.15 105.452) (end 143.258 106.559) (width 0.2) (layer "B.Cu") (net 4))
 (segment (start 131.732 100.3) (end 134.53 100.3) (width 0.2) (layer "F.Cu") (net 25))
 (segment (start 113.82 94.31) (end 125.742 94.31) (width 0.2) (layer "F.Cu") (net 25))
 (segment (start 125.742 94.31) (end 131.732 100.3) (width 0.2) (layer "F.Cu") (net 25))
 (segment (start 142.15 111.348) (end 142.15 112.45) (width 0.2) (layer "B.Cu") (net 25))
 (segment (start 140.999 106.769) (end 140.999 110.198) (width 0.2) (layer "B.Cu") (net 25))
 (segment (start 141 110.198) (end 142.15 111.348) (width 0.2) (layer "B.Cu") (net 25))
 (segment (start 134.53 100.3) (end 140.999 106.769) (width 0.2) (layer "B.Cu") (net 25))
 (segment (start 140.999 110.198) (end 141 110.198) (width 0.2) (layer "B.Cu") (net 25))
 (segment (start 131.826 101.646) (end 131.826 85.1619) (width 0.2) (layer "B.Cu") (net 6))
 (segment (start 131.826 85.1619) (end 118.115 71.45) (width 0.2) (layer "B.Cu") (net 6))
 (segment (start 118.115 71.45) (end 113.82 71.45) (width 0.2) (layer "B.Cu") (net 6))
 (segment (start 134.53 104.35) (end 131.826 101.646) (width 0.2) (layer "B.Cu") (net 6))
 (segment (start 135.7529 70) (end 136.091 70.3381) (width 0.2) (layer "F.Cu") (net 8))
 (segment (start 107.302 71.45) (end 108.752 70) (width 0.2) (layer "F.Cu") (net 8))
 (segment (start 108.752 70) (end 135.7529 70) (width 0.2) (layer "F.Cu") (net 8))
 (segment (start 106.2 71.45) (end 107.302 71.45) (width 0.2) (layer "F.Cu") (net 8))
 (via (at 136.091 70.3381) (size 0.6) (drill 0.3) (layers "F.Cu" "B.Cu") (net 8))
 (segment (start 142.15 107.298) (end 142.15 108.4) (width 0.2) (layer "B.Cu") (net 8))
 (segment (start 140.506 74.753) (end 140.506 105.654) (width 0.2) (layer "B.Cu") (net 8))
 (segment (start 140.506 105.654) (end 142.15 107.298) (width 0.2) (layer "B.Cu") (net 8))
 (segment (start 136.091 70.3381) (end 140.506 74.753) (width 0.2) (layer "B.Cu") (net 8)))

